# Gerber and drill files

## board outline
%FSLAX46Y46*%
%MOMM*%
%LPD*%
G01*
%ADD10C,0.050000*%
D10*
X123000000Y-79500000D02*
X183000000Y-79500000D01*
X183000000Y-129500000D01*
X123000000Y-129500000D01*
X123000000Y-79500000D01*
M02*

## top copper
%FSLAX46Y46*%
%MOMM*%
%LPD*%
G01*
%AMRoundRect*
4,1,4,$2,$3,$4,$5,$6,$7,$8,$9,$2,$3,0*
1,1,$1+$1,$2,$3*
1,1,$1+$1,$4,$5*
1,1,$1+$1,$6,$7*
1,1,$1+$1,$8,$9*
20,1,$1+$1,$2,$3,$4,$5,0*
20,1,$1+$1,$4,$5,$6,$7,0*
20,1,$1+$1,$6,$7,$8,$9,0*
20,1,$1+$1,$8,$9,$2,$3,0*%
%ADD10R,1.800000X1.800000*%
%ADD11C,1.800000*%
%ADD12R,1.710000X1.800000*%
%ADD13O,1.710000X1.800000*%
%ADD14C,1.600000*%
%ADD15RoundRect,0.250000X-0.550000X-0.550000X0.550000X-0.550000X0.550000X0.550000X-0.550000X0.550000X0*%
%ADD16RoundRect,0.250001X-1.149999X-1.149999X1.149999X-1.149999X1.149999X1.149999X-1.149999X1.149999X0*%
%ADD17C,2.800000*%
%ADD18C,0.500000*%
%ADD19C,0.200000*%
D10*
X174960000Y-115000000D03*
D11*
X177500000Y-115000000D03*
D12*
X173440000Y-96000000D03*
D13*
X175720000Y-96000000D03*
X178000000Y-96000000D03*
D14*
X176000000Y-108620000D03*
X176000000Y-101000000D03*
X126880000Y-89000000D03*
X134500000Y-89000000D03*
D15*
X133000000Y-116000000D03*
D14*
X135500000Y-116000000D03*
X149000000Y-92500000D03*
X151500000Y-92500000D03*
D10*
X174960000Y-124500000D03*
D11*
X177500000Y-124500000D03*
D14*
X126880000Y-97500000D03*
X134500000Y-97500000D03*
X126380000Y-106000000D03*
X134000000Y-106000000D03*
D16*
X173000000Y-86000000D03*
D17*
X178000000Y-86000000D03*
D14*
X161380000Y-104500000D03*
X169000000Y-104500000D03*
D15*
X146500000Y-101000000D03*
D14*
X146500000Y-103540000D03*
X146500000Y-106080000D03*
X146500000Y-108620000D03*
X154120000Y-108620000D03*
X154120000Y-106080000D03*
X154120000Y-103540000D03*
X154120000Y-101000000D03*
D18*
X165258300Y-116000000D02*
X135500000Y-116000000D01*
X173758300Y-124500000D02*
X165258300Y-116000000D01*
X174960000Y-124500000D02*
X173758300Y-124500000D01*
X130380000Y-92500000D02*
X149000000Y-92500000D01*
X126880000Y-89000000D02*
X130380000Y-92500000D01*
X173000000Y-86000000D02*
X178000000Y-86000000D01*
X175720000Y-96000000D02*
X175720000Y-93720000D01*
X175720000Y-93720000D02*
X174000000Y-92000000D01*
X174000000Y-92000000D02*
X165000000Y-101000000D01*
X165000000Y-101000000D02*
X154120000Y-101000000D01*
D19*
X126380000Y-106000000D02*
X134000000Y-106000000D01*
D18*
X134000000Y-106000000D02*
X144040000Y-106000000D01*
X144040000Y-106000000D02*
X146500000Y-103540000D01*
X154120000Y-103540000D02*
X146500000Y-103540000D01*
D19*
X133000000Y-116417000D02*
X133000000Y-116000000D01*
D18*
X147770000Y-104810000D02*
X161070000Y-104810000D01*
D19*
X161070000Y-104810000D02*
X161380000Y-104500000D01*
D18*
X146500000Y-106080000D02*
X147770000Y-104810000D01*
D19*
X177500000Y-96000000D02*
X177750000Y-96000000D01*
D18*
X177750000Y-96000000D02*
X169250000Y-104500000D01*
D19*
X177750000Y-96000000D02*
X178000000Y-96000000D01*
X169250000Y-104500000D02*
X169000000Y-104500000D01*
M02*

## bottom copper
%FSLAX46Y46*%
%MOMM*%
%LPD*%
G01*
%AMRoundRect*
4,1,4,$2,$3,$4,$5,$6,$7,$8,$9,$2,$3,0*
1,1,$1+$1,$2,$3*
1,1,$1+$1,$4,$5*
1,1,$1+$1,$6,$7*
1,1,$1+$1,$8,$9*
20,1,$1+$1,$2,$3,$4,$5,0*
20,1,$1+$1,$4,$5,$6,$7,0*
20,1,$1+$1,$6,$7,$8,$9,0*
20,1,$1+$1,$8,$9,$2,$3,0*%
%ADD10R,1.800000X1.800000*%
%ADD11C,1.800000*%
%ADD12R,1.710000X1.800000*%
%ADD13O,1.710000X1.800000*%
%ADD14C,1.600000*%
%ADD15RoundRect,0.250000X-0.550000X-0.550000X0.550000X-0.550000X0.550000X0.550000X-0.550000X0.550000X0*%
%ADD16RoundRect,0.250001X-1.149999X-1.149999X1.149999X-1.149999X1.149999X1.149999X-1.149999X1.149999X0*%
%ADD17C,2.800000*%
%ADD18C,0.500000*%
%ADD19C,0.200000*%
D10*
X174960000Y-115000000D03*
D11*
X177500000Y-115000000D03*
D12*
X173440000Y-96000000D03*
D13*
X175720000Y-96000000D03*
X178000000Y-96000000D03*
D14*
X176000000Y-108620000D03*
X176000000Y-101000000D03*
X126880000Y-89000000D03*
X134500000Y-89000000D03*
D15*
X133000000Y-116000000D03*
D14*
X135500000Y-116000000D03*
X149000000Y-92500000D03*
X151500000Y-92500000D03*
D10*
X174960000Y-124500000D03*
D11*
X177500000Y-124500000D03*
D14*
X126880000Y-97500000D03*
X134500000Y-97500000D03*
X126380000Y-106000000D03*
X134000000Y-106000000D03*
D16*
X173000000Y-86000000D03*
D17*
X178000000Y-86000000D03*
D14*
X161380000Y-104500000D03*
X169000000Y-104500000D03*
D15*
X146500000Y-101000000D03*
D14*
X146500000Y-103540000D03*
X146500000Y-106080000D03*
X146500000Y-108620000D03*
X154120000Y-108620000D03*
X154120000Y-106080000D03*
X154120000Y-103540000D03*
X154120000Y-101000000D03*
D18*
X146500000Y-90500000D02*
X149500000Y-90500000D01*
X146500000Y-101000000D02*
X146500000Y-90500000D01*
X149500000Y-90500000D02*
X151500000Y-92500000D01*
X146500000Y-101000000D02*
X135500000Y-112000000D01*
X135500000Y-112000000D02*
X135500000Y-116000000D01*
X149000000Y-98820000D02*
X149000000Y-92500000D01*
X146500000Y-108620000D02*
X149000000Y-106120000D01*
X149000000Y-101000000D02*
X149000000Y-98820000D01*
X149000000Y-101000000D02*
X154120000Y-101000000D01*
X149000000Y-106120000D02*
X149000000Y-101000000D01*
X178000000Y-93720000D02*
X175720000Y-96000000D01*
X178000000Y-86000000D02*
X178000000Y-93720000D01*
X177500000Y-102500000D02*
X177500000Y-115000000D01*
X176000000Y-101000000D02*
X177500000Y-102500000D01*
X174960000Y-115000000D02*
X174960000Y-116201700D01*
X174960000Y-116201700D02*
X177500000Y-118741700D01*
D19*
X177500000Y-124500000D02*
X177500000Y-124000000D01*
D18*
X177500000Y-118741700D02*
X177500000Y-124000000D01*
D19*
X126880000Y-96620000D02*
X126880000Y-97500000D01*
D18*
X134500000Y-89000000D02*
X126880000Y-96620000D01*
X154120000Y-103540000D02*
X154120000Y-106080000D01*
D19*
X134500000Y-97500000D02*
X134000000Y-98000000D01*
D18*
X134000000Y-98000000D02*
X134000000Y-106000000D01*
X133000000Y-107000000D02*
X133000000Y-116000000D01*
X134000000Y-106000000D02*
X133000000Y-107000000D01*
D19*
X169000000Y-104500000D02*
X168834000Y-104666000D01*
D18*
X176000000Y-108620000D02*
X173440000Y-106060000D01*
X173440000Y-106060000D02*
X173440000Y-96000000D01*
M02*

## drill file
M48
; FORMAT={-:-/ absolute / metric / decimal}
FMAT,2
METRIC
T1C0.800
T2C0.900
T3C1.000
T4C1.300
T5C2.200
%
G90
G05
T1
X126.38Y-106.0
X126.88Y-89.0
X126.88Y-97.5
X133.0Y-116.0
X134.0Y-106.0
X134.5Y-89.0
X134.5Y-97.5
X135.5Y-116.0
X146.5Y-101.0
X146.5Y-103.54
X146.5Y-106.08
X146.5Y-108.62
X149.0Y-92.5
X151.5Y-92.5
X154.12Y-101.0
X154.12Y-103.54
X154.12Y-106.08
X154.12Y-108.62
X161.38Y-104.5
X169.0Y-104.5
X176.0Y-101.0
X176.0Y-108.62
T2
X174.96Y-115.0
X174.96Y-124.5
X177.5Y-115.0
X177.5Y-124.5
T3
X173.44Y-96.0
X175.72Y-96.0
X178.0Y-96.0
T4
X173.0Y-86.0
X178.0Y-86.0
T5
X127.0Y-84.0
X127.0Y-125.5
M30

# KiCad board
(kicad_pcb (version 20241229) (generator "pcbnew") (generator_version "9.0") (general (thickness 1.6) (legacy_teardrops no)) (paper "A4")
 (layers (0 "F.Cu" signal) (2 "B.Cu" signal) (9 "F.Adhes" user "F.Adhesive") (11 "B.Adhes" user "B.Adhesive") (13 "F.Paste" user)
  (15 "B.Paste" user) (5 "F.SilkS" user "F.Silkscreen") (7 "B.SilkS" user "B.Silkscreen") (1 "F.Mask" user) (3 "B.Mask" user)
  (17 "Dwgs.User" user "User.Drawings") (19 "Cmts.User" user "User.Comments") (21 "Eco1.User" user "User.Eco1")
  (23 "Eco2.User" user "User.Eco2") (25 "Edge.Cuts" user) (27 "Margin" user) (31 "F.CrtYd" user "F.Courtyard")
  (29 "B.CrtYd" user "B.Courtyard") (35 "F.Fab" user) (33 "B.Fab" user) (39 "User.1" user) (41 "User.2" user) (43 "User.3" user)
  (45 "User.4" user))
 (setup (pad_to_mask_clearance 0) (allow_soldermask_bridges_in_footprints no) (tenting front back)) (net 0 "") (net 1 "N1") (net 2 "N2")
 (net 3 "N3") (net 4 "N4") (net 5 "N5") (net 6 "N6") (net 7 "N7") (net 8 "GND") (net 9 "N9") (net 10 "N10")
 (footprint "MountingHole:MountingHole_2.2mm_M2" (layer "F.Cu") (at 127 84)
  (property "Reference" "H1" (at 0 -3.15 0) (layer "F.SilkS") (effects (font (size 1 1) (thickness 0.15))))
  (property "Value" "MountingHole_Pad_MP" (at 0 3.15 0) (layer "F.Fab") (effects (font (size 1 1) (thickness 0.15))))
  (pad "" np_thru_hole circle (at 0 0) (size 2.2 2.2) (drill 2.2) (layers "*.Cu" "*.Mask")))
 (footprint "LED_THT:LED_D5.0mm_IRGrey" (layer "F.Cu") (at 174.96 115)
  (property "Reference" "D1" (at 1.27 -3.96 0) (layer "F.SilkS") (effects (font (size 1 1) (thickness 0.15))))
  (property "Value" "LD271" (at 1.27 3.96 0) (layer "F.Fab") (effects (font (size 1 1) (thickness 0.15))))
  (pad "1" thru_hole rect (at 0 0) (size 1.8 1.8) (drill 0.9) (layers "*.Cu" "*.Mask") (remove_unused_layers no) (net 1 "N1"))
  (pad "2" thru_hole circle (at 2.54 0) (size 1.8 1.8) (drill 0.9) (layers "*.Cu" "*.Mask") (remove_unused_layers no) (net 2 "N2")))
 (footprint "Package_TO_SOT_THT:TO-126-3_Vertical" (layer "F.Cu") (at 173.44 96)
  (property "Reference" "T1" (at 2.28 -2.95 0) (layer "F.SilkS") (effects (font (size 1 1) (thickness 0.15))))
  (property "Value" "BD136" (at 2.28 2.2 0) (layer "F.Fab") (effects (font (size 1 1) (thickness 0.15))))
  (pad "1" thru_hole rect (at 0 0) (size 1.71 1.8) (drill 1) (layers "*.Cu" "*.Mask") (remove_unused_layers no) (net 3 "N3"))
  (pad "2" thru_hole oval (at 2.28 0) (size 1.71 1.8) (drill 1) (layers "*.Cu" "*.Mask") (remove_unused_layers no) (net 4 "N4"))
  (pad "3" thru_hole oval (at 4.56 0) (size 1.71 1.8) (drill 1) (layers "*.Cu" "*.Mask") (remove_unused_layers no) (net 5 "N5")))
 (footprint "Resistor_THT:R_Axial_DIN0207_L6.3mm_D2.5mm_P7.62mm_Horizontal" (layer "F.Cu") (at 176 108.62 90)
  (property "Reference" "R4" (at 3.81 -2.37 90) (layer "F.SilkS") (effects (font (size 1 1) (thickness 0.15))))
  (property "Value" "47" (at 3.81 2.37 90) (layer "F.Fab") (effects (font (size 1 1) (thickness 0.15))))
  (pad "1" thru_hole circle (at 0 0 90) (size 1.6 1.6) (drill 0.8) (layers "*.Cu" "*.Mask") (remove_unused_layers no) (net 3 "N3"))
  (pad "2" thru_hole circle (at 7.62 0 90) (size 1.6 1.6) (drill 0.8) (layers "*.Cu" "*.Mask") (remove_unused_layers no) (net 2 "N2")))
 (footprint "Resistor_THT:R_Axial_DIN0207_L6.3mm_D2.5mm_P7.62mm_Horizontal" (layer "F.Cu") (at 126.88 89)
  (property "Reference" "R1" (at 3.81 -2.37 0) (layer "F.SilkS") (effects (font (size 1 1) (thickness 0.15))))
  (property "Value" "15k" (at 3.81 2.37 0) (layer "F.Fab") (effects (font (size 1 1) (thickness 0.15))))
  (pad "1" thru_hole circle (at 0 0) (size 1.6 1.6) (drill 0.8) (layers "*.Cu" "*.Mask") (remove_unused_layers no) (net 4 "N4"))
  (pad "2" thru_hole circle (at 7.62 0) (size 1.6 1.6) (drill 0.8) (layers "*.Cu" "*.Mask") (remove_unused_layers no) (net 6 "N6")))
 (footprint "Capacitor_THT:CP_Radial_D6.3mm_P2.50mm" (layer "F.Cu") (at 133 116)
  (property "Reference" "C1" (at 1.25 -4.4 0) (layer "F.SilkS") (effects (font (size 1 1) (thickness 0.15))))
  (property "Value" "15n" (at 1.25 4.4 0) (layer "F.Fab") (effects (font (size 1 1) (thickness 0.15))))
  (pad "1" thru_hole roundrect (at 0 0) (size 1.6 1.6) (drill 0.8) (layers "*.Cu" "*.Mask") (remove_unused_layers no)
   (roundrect_rratio 0.15625) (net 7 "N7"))
  (pad "2" thru_hole circle (at 2.5 0) (size 1.6 1.6) (drill 0.8) (layers "*.Cu" "*.Mask") (remove_unused_layers no) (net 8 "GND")))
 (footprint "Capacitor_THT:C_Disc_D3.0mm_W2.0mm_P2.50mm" (layer "F.Cu") (at 149 92.5)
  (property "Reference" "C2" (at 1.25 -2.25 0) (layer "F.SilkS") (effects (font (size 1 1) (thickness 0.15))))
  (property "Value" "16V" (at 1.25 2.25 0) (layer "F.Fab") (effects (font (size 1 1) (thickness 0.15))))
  (pad "1" thru_hole circle (at 0 0) (size 1.6 1.6) (drill 0.8) (layers "*.Cu" "*.Mask") (remove_unused_layers no) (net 4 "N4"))
  (pad "2" thru_hole circle (at 2.5 0) (size 1.6 1.6) (drill 0.8) (layers "*.Cu" "*.Mask") (remove_unused_layers no) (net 8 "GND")))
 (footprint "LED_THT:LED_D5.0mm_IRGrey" (layer "F.Cu") (at 174.96 124.5)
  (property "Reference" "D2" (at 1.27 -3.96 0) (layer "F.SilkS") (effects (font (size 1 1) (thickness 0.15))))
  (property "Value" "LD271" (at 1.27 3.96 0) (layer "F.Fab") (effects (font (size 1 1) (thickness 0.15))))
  (pad "1" thru_hole rect (at 0 0) (size 1.8 1.8) (drill 0.9) (layers "*.Cu" "*.Mask") (remove_unused_layers no) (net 8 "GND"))
  (pad "2" thru_hole circle (at 2.54 0) (size 1.8 1.8) (drill 0.9) (layers "*.Cu" "*.Mask") (remove_unused_layers no) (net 1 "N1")))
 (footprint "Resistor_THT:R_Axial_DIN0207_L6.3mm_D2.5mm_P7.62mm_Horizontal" (layer "F.Cu") (at 126.88 97.5)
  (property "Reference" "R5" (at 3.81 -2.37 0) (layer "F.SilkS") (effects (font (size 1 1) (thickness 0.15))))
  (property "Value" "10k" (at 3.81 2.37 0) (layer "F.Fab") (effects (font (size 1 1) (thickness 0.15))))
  (pad "1" thru_hole circle (at 0 0) (size 1.6 1.6) (drill 0.8) (layers "*.Cu" "*.Mask") (remove_unused_layers no) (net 6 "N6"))
  (pad "2" thru_hole circle (at 7.62 0) (size 1.6 1.6) (drill 0.8) (layers "*.Cu" "*.Mask") (remove_unused_layers no) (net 7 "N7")))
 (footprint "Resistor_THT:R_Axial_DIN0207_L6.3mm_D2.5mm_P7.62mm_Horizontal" (layer "F.Cu") (at 126.38 106)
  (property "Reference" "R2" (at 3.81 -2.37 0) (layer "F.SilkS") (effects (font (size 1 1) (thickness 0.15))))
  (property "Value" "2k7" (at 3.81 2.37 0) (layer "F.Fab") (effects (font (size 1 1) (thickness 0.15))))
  (pad "1" thru_hole circle (at 0 0) (size 1.6 1.6) (drill 0.8) (layers "*.Cu" "*.Mask") (remove_unused_layers no) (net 7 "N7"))
  (pad "2" thru_hole circle (at 7.62 0) (size 1.6 1.6) (drill 0.8) (layers "*.Cu" "*.Mask") (remove_unused_layers no) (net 7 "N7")))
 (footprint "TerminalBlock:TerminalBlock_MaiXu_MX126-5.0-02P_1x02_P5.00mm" (layer "F.Cu") (at 173 86)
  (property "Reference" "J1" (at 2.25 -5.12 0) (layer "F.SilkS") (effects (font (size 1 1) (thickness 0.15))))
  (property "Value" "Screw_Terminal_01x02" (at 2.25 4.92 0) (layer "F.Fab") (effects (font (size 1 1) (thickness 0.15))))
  (pad "1" thru_hole roundrect (at 0 0) (size 2.8 2.8) (drill 1.3) (layers "*.Cu" "*.Mask") (remove_unused_layers no)
   (roundrect_rratio 0.089286) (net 4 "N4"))
  (pad "2" thru_hole circle (at 5 0) (size 2.8 2.8) (drill 1.3) (layers "*.Cu" "*.Mask") (remove_unused_layers no) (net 4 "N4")))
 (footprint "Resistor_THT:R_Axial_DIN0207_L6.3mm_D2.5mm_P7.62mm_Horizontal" (layer "F.Cu") (at 161.38 104.5)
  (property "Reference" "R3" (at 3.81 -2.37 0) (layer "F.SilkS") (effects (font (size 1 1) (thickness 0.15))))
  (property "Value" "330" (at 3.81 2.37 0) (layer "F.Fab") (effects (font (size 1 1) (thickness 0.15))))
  (pad "1" thru_hole circle (at 0 0) (size 1.6 1.6) (drill 0.8) (layers "*.Cu" "*.Mask") (remove_unused_layers no) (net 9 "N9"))
  (pad "2" thru_hole circle (at 7.62 0) (size 1.6 1.6) (drill 0.8) (layers "*.Cu" "*.Mask") (remove_unused_layers no) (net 5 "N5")))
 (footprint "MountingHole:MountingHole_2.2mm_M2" (layer "F.Cu") (at 127 125.5)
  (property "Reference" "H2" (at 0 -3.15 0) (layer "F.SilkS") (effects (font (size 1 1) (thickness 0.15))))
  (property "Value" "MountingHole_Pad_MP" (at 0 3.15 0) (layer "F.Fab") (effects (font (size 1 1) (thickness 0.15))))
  (pad "" np_thru_hole circle (at 0 0) (size 2.2 2.2) (drill 2.2) (layers "*.Cu" "*.Mask")))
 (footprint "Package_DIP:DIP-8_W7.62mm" (layer "F.Cu") (at 146.5 101)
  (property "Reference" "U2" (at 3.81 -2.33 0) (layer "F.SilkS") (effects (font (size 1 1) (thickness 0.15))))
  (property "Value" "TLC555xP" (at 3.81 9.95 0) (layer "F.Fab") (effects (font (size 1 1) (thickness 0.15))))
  (pad "1" thru_hole roundrect (at 0 0) (size 1.6 1.6) (drill 0.8) (layers "*.Cu" "*.Mask") (remove_unused_layers no)
   (roundrect_rratio 0.15625) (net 8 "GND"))
  (pad "2" thru_hole circle (at 0 2.54) (size 1.6 1.6) (drill 0.8) (layers "*.Cu" "*.Mask") (remove_unused_layers no) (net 7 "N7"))
  (pad "3" thru_hole circle (at 0 5.08) (size 1.6 1.6) (drill 0.8) (layers "*.Cu" "*.Mask") (remove_unused_layers no) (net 9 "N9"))
  (pad "4" thru_hole circle (at 0 7.62) (size 1.6 1.6) (drill 0.8) (layers "*.Cu" "*.Mask") (remove_unused_layers no) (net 4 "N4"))
  (pad "5" thru_hole circle (at 7.62 7.62) (size 1.6 1.6) (drill 0.8) (layers "*.Cu" "*.Mask") (remove_unused_layers no) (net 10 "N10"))
  (pad "6" thru_hole circle (at 7.62 5.08) (size 1.6 1.6) (drill 0.8) (layers "*.Cu" "*.Mask") (remove_unused_layers no) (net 7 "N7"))
  (pad "7" thru_hole circle (at 7.62 2.54) (size 1.6 1.6) (drill 0.8) (layers "*.Cu" "*.Mask") (remove_unused_layers no) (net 7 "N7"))
  (pad "8" thru_hole circle (at 7.62 0) (size 1.6 1.6) (drill 0.8) (layers "*.Cu" "*.Mask") (remove_unused_layers no) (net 4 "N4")))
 (gr_rect (start 123 79.5) (end 183 129.5) (stroke (width 0.05) (type solid)) (fill no) (layer "Edge.Cuts"))
 (segment (start 165.2583 116) (end 135.5 116) (width 0.5) (layer "F.Cu") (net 8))
 (segment (start 173.7583 124.5) (end 165.2583 116) (width 0.5) (layer "F.Cu") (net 8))
 (segment (start 174.96 124.5) (end 173.7583 124.5) (width 0.5) (layer "F.Cu") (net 8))
 (segment (start 146.5 90.5) (end 149.5 90.5) (width 0.5) (layer "B.Cu") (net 8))
 (segment (start 146.5 101) (end 146.5 90.5) (width 0.5) (layer "B.Cu") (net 8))
 (segment (start 149.5 90.5) (end 151.5 92.5) (width 0.5) (layer "B.Cu") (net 8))
 (segment (start 146.5 101) (end 135.5 112) (width 0.5) (layer "B.Cu") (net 8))
 (segment (start 135.5 112) (end 135.5 116) (width 0.5) (layer "B.Cu") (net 8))
 (segment (start 130.38 92.5) (end 149 92.5) (width 0.5) (layer "F.Cu") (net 4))
 (segment (start 126.88 89) (end 130.38 92.5) (width 0.5) (layer "F.Cu") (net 4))
 (segment (start 173 86) (end 178 86) (width 0.5) (layer "F.Cu") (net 4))
 (segment (start 175.72 96) (end 175.72 93.72) (width 0.5) (layer "F.Cu") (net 4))
 (segment (start 175.72 93.72) (end 174 92) (width 0.5) (layer "F.Cu") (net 4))
 (segment (start 174 92) (end 165 101) (width 0.5) (layer "F.Cu") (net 4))
 (segment (start 165 101) (end 154.12 101) (width 0.5) (layer "F.Cu") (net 4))
 (segment (start 149 98.82) (end 149 92.5) (width 0.5) (layer "B.Cu") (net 4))
 (segment (start 146.5 108.62) (end 149 106.12) (width 0.5) (layer "B.Cu") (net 4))
 (segment (start 149 101) (end 149 98.82) (width 0.5) (layer "B.Cu") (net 4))
 (segment (start 149 101) (end 154.12 101) (width 0.5) (layer "B.Cu") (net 4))
 (segment (start 149 106.12) (end 149 101) (width 0.5) (layer "B.Cu") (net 4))
 (segment (start 178 93.72) (end 175.72 96) (width 0.5) (layer "B.Cu") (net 4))
 (segment (start 178 86) (end 178 93.72) (width 0.5) (layer "B.Cu") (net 4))
 (segment (start 177.5 102.5) (end 177.5 115) (width 0.5) (layer "B.Cu") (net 2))
 (segment (start 176 101) (end 177.5 102.5) (width 0.5) (layer "B.Cu") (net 2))
 (segment (start 174.96 115) (end 174.96 116.2017) (width 0.5) (layer "B.Cu") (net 1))
 (segment (start 174.96 116.2017) (end 177.5 118.7417) (width 0.5) (layer "B.Cu") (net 1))
 (segment (start 177.5 124.5) (end 177.5 124) (width 0.2) (layer "B.Cu") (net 1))
 (segment (start 177.5 118.7417) (end 177.5 124) (width 0.5) (layer "B.Cu") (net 1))
 (segment (start 126.88 96.62) (end 126.88 97.5) (width 0.2) (layer "B.Cu") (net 6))
 (segment (start 134.5 89) (end 126.88 96.62) (width 0.5) (layer "B.Cu") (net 6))
 (segment (start 126.38 106) (end 134 106) (width 0.2) (layer "F.Cu") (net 7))
 (segment (start 134 106) (end 144.04 106) (width 0.5) (layer "F.Cu") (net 7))
 (segment (start 144.04 106) (end 146.5 103.54) (width 0.5) (layer "F.Cu") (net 7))
 (segment (start 154.12 103.54) (end 146.5 103.54) (width 0.5) (layer "F.Cu") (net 7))
 (segment (start 133 116.417) (end 133 116) (width 0.2) (layer "F.Cu") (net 7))
 (segment (start 154.12 103.54) (end 154.12 106.08) (width 0.5) (layer "B.Cu") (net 7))
 (segment (start 134.5 97.5) (end 134 98) (width 0.2) (layer "B.Cu") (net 7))
 (segment (start 134 98) (end 134 106) (width 0.5) (layer "B.Cu") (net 7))
 (segment (start 133 107) (end 133 116) (width 0.5) (layer "B.Cu") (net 7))
 (segment (start 134 106) (end 133 107) (width 0.5) (layer "B.Cu") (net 7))
 (segment (start 147.77 104.81) (end 161.07 104.81) (width 0.5) (layer "F.Cu") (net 9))
 (segment (start 161.07 104.81) (end 161.38 104.5) (width 0.2) (layer "F.Cu") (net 9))
 (segment (start 146.5 106.08) (end 147.77 104.81) (width 0.5) (layer "F.Cu") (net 9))
 (segment (start 177.5 96) (end 177.75 96) (width 0.2) (layer "F.Cu") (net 5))
 (segment (start 177.75 96) (end 169.25 104.5) (width 0.5) (layer "F.Cu") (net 5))
 (segment (start 177.75 96) (end 178 96) (width 0.2) (layer "F.Cu") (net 5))
 (segment (start 169.25 104.5) (end 169 104.5) (width 0.2) (layer "F.Cu") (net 5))
 (segment (start 169 104.5) (end 168.834 104.666) (width 0.2) (layer "B.Cu") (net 5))
 (segment (start 176 108.62) (end 173.44 106.06) (width 0.5) (layer "B.Cu") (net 3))
 (segment (start 173.44 106.06) (end 173.44 96) (width 0.5) (layer "B.Cu") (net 3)))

